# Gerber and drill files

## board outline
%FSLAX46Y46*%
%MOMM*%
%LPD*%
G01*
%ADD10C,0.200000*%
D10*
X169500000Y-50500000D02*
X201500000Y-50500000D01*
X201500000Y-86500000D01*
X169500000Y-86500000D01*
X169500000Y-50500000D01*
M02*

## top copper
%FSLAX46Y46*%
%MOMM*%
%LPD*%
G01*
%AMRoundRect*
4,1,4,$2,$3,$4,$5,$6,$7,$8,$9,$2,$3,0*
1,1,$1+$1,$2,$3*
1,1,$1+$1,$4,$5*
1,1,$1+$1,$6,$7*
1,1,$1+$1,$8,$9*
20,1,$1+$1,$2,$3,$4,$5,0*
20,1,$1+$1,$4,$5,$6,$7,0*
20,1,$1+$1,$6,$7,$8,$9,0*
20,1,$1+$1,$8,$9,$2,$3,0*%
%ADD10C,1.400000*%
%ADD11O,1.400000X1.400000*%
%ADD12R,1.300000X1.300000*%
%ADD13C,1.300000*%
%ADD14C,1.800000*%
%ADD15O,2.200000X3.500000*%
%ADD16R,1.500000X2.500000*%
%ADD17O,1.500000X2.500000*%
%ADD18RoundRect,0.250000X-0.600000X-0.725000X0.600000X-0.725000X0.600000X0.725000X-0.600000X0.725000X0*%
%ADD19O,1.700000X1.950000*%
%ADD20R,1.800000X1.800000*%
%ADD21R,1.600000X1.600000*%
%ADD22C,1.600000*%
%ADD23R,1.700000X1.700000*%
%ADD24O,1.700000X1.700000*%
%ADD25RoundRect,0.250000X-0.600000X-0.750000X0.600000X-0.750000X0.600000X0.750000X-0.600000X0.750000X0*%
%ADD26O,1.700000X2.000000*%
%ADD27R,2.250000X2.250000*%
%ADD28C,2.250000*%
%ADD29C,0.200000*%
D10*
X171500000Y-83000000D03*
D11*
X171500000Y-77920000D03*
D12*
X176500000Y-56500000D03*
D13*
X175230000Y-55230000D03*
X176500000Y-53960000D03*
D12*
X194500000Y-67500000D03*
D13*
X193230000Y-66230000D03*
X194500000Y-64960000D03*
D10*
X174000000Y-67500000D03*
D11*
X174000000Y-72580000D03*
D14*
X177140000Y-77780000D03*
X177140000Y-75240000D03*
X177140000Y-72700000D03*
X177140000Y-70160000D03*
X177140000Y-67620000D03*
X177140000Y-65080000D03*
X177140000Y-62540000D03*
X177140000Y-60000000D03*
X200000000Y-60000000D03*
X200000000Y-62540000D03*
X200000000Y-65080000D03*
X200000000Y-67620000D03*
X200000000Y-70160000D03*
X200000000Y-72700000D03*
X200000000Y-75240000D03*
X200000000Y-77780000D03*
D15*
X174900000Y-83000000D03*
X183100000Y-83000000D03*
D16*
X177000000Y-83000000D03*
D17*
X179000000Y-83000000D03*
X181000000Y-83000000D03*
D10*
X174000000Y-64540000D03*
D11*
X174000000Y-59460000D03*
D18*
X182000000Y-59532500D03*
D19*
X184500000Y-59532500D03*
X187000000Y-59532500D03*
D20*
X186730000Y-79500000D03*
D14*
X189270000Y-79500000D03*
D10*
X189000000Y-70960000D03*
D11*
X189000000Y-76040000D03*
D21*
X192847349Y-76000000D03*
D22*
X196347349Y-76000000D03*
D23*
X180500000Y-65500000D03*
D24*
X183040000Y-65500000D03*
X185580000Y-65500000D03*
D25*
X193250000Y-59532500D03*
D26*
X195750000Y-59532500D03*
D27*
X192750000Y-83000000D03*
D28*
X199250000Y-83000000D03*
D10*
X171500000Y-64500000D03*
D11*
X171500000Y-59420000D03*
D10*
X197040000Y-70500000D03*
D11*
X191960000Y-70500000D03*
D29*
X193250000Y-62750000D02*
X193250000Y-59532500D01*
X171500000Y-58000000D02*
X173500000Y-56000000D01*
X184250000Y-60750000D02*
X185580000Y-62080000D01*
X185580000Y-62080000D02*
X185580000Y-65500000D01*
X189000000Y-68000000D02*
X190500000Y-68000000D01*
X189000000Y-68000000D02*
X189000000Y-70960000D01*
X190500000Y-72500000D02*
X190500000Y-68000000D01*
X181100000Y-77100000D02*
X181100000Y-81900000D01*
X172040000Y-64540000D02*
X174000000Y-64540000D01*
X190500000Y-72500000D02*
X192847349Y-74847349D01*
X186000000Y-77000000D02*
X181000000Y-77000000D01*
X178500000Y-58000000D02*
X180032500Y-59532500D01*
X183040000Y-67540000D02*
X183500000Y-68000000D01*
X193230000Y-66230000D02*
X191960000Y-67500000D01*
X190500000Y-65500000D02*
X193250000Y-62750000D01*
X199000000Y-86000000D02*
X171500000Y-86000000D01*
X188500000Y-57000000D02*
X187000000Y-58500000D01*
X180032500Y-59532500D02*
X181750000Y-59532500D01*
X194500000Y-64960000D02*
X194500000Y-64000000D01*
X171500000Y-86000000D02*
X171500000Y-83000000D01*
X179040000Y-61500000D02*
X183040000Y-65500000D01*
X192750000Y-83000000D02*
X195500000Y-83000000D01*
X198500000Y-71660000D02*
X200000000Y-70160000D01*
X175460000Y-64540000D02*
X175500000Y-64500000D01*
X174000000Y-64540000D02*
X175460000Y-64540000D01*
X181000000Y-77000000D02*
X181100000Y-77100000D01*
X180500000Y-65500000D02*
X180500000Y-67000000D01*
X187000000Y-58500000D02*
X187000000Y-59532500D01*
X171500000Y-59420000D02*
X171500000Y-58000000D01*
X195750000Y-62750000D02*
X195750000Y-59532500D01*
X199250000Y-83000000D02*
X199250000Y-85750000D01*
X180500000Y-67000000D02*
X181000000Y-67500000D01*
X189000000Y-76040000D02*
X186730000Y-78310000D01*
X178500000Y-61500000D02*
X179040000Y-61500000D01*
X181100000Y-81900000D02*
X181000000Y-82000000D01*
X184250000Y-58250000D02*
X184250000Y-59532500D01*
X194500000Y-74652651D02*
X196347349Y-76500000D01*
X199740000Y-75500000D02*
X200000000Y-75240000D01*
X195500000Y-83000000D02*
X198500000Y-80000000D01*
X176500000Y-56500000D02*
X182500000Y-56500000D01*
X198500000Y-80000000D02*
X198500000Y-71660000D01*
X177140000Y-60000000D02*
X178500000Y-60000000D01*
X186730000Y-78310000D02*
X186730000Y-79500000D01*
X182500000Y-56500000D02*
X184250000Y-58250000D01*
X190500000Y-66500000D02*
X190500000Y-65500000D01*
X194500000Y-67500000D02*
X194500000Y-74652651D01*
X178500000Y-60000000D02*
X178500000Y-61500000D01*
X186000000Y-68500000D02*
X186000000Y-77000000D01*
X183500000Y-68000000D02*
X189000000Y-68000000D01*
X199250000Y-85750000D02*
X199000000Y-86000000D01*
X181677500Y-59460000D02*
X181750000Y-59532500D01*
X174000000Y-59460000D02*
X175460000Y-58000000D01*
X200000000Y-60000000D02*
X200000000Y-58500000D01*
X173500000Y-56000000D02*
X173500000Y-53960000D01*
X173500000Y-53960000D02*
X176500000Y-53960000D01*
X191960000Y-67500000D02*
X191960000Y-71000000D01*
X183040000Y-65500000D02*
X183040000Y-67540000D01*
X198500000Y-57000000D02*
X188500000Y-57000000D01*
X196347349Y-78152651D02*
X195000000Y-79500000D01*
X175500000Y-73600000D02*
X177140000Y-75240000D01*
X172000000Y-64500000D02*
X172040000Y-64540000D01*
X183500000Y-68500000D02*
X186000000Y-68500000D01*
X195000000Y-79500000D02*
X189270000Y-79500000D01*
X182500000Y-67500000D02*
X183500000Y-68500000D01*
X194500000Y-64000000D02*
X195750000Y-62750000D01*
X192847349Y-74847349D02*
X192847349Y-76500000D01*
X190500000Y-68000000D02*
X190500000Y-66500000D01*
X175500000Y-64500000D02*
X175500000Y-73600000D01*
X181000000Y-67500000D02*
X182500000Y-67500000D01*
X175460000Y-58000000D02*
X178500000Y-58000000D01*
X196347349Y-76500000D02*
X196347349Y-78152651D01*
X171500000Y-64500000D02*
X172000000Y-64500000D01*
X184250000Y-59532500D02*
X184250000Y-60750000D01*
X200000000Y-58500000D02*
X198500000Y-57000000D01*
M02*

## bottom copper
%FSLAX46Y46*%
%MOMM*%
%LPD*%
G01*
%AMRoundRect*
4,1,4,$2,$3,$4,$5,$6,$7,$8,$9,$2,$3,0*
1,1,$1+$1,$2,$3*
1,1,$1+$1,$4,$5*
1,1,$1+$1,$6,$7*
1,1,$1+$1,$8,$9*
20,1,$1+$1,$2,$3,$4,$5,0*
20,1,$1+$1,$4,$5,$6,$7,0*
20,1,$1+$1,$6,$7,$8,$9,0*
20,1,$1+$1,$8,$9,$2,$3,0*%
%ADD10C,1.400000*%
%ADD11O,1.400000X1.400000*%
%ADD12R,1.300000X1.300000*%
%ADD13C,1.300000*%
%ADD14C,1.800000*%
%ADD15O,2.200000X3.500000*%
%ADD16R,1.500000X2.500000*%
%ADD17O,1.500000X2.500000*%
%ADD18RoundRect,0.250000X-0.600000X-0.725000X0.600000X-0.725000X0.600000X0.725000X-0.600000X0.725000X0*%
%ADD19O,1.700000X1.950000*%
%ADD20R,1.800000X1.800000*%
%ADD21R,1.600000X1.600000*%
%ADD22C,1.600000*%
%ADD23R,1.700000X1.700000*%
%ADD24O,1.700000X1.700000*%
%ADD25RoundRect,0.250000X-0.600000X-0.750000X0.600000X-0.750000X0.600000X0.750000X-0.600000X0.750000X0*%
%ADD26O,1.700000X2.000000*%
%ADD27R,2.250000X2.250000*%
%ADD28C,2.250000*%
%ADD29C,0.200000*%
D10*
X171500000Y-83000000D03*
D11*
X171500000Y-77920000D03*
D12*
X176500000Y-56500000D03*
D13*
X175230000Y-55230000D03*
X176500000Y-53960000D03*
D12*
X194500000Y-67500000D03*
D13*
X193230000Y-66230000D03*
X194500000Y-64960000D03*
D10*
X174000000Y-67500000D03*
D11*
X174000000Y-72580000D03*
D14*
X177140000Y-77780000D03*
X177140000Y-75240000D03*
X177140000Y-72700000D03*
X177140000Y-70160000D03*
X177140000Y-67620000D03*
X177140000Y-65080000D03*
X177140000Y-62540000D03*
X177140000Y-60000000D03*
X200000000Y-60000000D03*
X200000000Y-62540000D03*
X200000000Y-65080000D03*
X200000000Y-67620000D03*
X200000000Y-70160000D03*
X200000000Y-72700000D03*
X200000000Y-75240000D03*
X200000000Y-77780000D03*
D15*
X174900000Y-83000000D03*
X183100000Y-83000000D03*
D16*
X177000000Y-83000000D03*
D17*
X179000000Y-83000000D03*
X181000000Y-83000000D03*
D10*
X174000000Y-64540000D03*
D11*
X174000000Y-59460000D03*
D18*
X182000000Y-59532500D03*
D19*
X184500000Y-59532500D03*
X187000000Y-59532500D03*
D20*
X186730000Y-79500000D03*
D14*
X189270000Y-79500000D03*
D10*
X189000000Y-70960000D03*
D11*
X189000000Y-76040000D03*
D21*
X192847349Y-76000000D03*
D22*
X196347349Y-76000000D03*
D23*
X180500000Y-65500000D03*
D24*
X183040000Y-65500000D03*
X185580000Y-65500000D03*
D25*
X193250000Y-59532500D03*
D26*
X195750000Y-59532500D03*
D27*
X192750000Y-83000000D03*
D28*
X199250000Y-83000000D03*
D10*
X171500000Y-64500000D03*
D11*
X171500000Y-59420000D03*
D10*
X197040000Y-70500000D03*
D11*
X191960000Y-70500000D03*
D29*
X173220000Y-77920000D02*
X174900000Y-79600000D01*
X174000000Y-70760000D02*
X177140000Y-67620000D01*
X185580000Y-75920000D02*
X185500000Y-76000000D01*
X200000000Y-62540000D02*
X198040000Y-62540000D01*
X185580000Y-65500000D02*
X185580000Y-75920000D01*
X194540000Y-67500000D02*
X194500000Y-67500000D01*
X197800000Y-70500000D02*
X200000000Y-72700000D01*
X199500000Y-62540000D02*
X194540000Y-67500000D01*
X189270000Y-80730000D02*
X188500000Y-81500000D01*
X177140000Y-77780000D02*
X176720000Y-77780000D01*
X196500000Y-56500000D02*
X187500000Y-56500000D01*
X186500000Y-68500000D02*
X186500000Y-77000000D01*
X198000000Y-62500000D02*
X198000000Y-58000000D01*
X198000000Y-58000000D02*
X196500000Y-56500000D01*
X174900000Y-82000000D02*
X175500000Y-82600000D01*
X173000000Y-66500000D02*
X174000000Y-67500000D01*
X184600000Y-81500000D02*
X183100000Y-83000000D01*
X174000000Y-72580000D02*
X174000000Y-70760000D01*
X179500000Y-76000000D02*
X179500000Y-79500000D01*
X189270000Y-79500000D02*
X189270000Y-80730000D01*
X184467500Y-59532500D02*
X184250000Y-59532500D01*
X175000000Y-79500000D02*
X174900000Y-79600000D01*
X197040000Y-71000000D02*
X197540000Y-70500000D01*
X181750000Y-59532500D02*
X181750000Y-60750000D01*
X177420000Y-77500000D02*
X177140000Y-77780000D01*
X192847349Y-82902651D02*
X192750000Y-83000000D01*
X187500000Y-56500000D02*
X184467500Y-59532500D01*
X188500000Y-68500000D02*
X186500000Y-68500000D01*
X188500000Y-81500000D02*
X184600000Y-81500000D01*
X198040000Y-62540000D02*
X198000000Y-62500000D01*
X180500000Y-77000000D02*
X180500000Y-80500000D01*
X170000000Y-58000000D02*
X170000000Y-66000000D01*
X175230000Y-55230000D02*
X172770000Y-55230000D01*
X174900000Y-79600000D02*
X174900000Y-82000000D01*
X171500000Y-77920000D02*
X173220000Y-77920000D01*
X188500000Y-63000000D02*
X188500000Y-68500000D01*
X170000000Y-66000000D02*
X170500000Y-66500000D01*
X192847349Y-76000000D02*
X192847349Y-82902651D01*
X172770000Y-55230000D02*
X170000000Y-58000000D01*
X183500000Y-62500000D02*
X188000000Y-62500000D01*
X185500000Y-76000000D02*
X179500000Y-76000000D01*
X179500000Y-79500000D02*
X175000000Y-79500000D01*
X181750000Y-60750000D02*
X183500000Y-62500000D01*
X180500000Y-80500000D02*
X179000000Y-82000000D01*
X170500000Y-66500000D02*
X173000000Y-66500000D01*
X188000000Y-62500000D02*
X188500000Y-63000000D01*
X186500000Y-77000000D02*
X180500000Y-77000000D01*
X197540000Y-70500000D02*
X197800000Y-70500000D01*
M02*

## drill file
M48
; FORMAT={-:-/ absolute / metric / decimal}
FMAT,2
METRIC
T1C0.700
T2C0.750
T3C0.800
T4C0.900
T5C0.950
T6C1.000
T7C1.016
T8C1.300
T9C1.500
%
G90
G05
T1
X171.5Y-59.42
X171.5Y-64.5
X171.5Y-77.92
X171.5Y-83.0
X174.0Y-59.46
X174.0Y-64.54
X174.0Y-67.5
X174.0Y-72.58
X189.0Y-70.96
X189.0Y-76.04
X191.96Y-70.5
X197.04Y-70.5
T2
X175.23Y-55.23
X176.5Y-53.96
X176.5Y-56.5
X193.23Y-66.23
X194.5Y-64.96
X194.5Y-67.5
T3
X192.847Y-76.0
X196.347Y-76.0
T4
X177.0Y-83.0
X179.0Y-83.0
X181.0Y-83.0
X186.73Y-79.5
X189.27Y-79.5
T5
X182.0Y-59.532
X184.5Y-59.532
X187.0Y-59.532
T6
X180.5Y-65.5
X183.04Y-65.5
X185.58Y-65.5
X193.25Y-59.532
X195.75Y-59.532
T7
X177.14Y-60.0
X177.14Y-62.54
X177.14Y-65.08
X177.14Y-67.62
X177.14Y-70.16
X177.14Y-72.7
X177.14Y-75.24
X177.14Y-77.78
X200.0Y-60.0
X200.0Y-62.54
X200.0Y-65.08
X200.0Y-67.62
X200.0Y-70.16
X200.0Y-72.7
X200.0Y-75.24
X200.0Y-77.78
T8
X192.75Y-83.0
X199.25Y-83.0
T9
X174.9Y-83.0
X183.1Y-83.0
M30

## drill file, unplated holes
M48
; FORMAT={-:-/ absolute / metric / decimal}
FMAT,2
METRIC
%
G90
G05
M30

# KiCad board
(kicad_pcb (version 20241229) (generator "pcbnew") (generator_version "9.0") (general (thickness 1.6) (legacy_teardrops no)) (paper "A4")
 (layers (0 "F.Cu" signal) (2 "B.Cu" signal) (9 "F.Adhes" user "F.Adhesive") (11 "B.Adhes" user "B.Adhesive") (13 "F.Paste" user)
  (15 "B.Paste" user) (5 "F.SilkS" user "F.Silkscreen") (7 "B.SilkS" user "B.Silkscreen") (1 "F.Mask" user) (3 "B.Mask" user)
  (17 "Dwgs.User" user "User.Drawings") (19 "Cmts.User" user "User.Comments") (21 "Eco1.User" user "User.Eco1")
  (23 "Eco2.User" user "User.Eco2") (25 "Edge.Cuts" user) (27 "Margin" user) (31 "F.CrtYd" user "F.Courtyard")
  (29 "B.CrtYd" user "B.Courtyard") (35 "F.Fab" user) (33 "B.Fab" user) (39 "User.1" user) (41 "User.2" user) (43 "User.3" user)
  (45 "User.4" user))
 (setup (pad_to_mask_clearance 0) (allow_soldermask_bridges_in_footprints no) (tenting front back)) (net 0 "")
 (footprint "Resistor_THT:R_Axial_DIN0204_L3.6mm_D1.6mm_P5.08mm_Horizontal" (layer "F.Cu") (at 171.5 83 90)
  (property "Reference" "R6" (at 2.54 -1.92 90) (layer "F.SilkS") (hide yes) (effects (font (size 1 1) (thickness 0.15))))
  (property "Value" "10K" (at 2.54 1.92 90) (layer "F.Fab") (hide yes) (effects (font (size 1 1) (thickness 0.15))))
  (pad "1" thru_hole circle (at 0 0 90) (size 1.4 1.4) (drill 0.7) (layers "*.Cu" "*.Mask") (remove_unused_layers no))
  (pad "2" thru_hole oval (at 5.08 0 90) (size 1.4 1.4) (drill 0.7) (layers "*.Cu" "*.Mask") (remove_unused_layers no)))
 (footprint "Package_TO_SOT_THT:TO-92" (layer "F.Cu") (at 176.5 56.5 90)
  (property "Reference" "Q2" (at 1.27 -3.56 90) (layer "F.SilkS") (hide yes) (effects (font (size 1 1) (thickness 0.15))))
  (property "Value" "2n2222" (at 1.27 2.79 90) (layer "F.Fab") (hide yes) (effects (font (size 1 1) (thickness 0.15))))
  (pad "1" thru_hole rect (at 0 0 90) (size 1.3 1.3) (drill 0.75) (layers "*.Cu" "*.Mask") (remove_unused_layers no))
  (pad "2" thru_hole circle (at 1.27 -1.27 90) (size 1.3 1.3) (drill 0.75) (layers "*.Cu" "*.Mask") (remove_unused_layers no))
  (pad "3" thru_hole circle (at 2.54 0 90) (size 1.3 1.3) (drill 0.75) (layers "*.Cu" "*.Mask") (remove_unused_layers no)))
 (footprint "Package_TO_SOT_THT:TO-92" (layer "F.Cu") (at 194.5 67.5 90)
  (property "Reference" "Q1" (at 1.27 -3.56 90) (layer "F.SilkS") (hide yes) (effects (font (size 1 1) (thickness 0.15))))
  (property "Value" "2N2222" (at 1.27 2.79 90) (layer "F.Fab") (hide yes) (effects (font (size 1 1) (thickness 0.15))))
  (pad "1" thru_hole rect (at 0 0 90) (size 1.3 1.3) (drill 0.75) (layers "*.Cu" "*.Mask") (remove_unused_layers no))
  (pad "2" thru_hole circle (at 1.27 -1.27 90) (size 1.3 1.3) (drill 0.75) (layers "*.Cu" "*.Mask") (remove_unused_layers no))
  (pad "3" thru_hole circle (at 2.54 0 90) (size 1.3 1.3) (drill 0.75) (layers "*.Cu" "*.Mask") (remove_unused_layers no)))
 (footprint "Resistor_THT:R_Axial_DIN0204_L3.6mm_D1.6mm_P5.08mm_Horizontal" (layer "F.Cu") (at 174 67.5 -90)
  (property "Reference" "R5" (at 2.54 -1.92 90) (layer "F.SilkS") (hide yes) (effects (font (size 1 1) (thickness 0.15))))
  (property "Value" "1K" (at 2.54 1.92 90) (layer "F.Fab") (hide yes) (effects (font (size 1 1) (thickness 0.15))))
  (pad "1" thru_hole circle (at 0 0 270) (size 1.4 1.4) (drill 0.7) (layers "*.Cu" "*.Mask") (remove_unused_layers no))
  (pad "2" thru_hole oval (at 5.08 0 270) (size 1.4 1.4) (drill 0.7) (layers "*.Cu" "*.Mask") (remove_unused_layers no)))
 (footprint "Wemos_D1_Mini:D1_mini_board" (layer "F.Cu") (at 188.57 70.16)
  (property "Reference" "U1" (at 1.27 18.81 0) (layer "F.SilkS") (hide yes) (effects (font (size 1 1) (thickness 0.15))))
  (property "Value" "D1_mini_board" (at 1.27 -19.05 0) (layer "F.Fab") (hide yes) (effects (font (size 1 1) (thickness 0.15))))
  (pad "1" thru_hole circle (at -11.43 7.62) (size 1.8 1.8) (drill 1.016) (layers "*.Cu" "*.Mask" "F.SilkS") (remove_unused_layers no))
  (pad "2" thru_hole circle (at -11.43 5.08) (size 1.8 1.8) (drill 1.016) (layers "*.Cu" "*.Mask" "F.SilkS") (remove_unused_layers no))
  (pad "3" thru_hole circle (at -11.43 2.54) (size 1.8 1.8) (drill 1.016) (layers "*.Cu" "*.Mask" "F.SilkS") (remove_unused_layers no))
  (pad "4" thru_hole circle (at -11.43 0) (size 1.8 1.8) (drill 1.016) (layers "*.Cu" "*.Mask" "F.SilkS") (remove_unused_layers no))
  (pad "5" thru_hole circle (at -11.43 -2.54) (size 1.8 1.8) (drill 1.016) (layers "*.Cu" "*.Mask" "F.SilkS") (remove_unused_layers no))
  (pad "6" thru_hole circle (at -11.43 -5.08) (size 1.8 1.8) (drill 1.016) (layers "*.Cu" "*.Mask" "F.SilkS") (remove_unused_layers no))
  (pad "7" thru_hole circle (at -11.43 -7.62) (size 1.8 1.8) (drill 1.016) (layers "*.Cu" "*.Mask" "F.SilkS") (remove_unused_layers no))
  (pad "8" thru_hole circle (at -11.43 -10.16) (size 1.8 1.8) (drill 1.016) (layers "*.Cu" "*.Mask" "F.SilkS") (remove_unused_layers no))
  (pad "9" thru_hole circle (at 11.43 -10.16) (size 1.8 1.8) (drill 1.016) (layers "*.Cu" "*.Mask" "F.SilkS") (remove_unused_layers no))
  (pad "10" thru_hole circle (at 11.43 -7.62) (size 1.8 1.8) (drill 1.016) (layers "*.Cu" "*.Mask" "F.SilkS") (remove_unused_layers no))
  (pad "11" thru_hole circle (at 11.43 -5.08) (size 1.8 1.8) (drill 1.016) (layers "*.Cu" "*.Mask" "F.SilkS") (remove_unused_layers no))
  (pad "12" thru_hole circle (at 11.43 -2.54) (size 1.8 1.8) (drill 1.016) (layers "*.Cu" "*.Mask" "F.SilkS") (remove_unused_layers no))
  (pad "13" thru_hole circle (at 11.43 0) (size 1.8 1.8) (drill 1.016) (layers "*.Cu" "*.Mask" "F.SilkS") (remove_unused_layers no))
  (pad "14" thru_hole circle (at 11.43 2.54) (size 1.8 1.8) (drill 1.016) (layers "*.Cu" "*.Mask" "F.SilkS") (remove_unused_layers no))
  (pad "15" thru_hole circle (at 11.43 5.08) (size 1.8 1.8) (drill 1.016) (layers "*.Cu" "*.Mask" "F.SilkS") (remove_unused_layers no))
  (pad "16" thru_hole circle (at 11.43 7.62) (size 1.8 1.8) (drill 1.016) (layers "*.Cu" "*.Mask" "F.SilkS") (remove_unused_layers no)))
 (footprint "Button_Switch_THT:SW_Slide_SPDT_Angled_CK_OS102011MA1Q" (layer "F.Cu") (at 177 83)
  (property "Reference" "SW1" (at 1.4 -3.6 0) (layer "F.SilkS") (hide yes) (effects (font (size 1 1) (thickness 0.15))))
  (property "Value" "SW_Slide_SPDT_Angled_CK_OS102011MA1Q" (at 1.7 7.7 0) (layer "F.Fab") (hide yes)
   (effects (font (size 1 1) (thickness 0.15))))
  (pad "" thru_hole oval (at -2.1 0) (size 2.2 3.5) (drill 1.5) (layers "*.Cu" "*.Mask") (remove_unused_layers no))
  (pad "" thru_hole oval (at 6.1 0) (size 2.2 3.5) (drill 1.5) (layers "*.Cu" "*.Mask") (remove_unused_layers no))
  (pad "1" thru_hole rect (at 0 0) (size 1.5 2.5) (drill 0.9) (layers "*.Cu" "*.Mask") (remove_unused_layers no))
  (pad "2" thru_hole oval (at 2 0) (size 1.5 2.5) (drill 0.9) (layers "*.Cu" "*.Mask") (remove_unused_layers no))
  (pad "3" thru_hole oval (at 4 0) (size 1.5 2.5) (drill 0.9) (layers "*.Cu" "*.Mask") (remove_unused_layers no)))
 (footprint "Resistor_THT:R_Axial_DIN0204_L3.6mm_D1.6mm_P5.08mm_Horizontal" (layer "F.Cu") (at 174 64.54 90)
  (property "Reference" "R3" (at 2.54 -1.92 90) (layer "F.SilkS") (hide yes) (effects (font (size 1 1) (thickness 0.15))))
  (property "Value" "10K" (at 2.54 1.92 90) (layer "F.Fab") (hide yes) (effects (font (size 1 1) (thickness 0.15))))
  (pad "1" thru_hole circle (at 0 0 90) (size 1.4 1.4) (drill 0.7) (layers "*.Cu" "*.Mask") (remove_unused_layers no))
  (pad "2" thru_hole oval (at 5.08 0 90) (size 1.4 1.4) (drill 0.7) (layers "*.Cu" "*.Mask") (remove_unused_layers no)))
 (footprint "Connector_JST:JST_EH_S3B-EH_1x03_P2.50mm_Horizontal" (layer "F.Cu") (at 182 59.5325)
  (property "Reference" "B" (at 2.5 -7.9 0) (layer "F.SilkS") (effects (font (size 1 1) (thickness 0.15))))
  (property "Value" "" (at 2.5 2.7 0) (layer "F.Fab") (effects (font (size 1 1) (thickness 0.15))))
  (pad "1" thru_hole roundrect (at 0 0) (size 1.7 1.95) (drill 0.95) (layers "*.Cu" "*.Mask") (remove_unused_layers no)
   (roundrect_rratio 0.147059))
  (pad "2" thru_hole oval (at 2.5 0) (size 1.7 1.95) (drill 0.95) (layers "*.Cu" "*.Mask") (remove_unused_layers no))
  (pad "3" thru_hole oval (at 5 0) (size 1.7 1.95) (drill 0.95) (layers "*.Cu" "*.Mask") (remove_unused_layers no)))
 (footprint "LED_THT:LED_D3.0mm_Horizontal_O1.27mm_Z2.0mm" (layer "F.Cu") (at 186.73 79.5)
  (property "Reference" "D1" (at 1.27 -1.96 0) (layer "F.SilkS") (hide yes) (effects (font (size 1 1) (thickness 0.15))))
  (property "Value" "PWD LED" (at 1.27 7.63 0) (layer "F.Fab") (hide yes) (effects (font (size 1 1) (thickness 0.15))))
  (pad "1" thru_hole rect (at 0 0) (size 1.8 1.8) (drill 0.9) (layers "*.Cu" "*.Mask") (remove_unused_layers no))
  (pad "2" thru_hole circle (at 2.54 0) (size 1.8 1.8) (drill 0.9) (layers "*.Cu" "*.Mask") (remove_unused_layers no)))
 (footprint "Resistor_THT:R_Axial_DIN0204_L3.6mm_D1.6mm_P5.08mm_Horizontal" (layer "F.Cu") (at 189 70.96 -90)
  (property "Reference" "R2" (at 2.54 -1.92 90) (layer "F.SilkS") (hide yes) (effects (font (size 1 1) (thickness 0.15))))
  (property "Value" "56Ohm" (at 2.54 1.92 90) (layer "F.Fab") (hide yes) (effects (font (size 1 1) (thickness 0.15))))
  (pad "1" thru_hole circle (at 0 0 270) (size 1.4 1.4) (drill 0.7) (layers "*.Cu" "*.Mask") (remove_unused_layers no))
  (pad "2" thru_hole oval (at 5.08 0 270) (size 1.4 1.4) (drill 0.7) (layers "*.Cu" "*.Mask") (remove_unused_layers no)))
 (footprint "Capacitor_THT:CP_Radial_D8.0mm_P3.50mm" (layer "F.Cu") (at 192.847349 76)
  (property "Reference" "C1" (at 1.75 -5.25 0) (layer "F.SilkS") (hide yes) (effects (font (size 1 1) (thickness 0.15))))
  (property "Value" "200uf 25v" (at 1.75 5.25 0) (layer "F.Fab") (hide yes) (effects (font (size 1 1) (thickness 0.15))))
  (pad "1" thru_hole rect (at 0 0) (size 1.6 1.6) (drill 0.8) (layers "*.Cu" "*.Mask") (remove_unused_layers no))
  (pad "2" thru_hole circle (at 3.5 0) (size 1.6 1.6) (drill 0.8) (layers "*.Cu" "*.Mask") (remove_unused_layers no)))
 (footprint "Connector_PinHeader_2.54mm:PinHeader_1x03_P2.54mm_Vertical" (layer "F.Cu") (at 180.5 65.5 90)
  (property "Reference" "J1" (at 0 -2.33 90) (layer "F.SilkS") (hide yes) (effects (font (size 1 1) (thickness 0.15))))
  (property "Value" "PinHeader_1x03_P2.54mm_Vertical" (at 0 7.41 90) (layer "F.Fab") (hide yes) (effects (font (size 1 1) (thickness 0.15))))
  (pad "1" thru_hole rect (at 0 0 90) (size 1.7 1.7) (drill 1) (layers "*.Cu" "*.Mask") (remove_unused_layers no))
  (pad "2" thru_hole oval (at 0 2.54 90) (size 1.7 1.7) (drill 1) (layers "*.Cu" "*.Mask") (remove_unused_layers no))
  (pad "3" thru_hole oval (at 0 5.08 90) (size 1.7 1.7) (drill 1) (layers "*.Cu" "*.Mask") (remove_unused_layers no)))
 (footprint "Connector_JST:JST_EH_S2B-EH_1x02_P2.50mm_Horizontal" (layer "F.Cu") (at 193.25 59.5325)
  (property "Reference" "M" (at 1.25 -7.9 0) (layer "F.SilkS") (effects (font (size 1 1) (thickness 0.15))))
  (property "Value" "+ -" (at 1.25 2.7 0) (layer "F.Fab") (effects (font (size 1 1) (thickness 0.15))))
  (pad "1" thru_hole roundrect (at 0 0) (size 1.7 2) (drill 1) (layers "*.Cu" "*.Mask") (remove_unused_layers no)
   (roundrect_rratio 0.147059))
  (pad "2" thru_hole oval (at 2.5 0) (size 1.7 2) (drill 1) (layers "*.Cu" "*.Mask") (remove_unused_layers no)))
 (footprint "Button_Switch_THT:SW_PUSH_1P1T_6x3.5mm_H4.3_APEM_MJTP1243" (layer "F.Cu") (at 192.75 83)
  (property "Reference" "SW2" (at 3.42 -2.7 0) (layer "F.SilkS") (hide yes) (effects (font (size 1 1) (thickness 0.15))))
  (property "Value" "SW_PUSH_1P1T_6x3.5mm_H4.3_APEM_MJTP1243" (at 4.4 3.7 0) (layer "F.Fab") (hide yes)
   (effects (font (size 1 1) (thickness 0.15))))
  (pad "1" thru_hole rect (at 0 0 90) (size 2.25 2.25) (drill 1.3) (layers "*.Cu" "*.Mask") (remove_unused_layers no))
  (pad "2" thru_hole circle (at 6.5 0 90) (size 2.25 2.25) (drill 1.3) (layers "*.Cu" "*.Mask") (remove_unused_layers no)))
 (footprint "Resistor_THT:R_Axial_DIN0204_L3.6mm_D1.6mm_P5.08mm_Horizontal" (layer "F.Cu") (at 171.5 64.5 90)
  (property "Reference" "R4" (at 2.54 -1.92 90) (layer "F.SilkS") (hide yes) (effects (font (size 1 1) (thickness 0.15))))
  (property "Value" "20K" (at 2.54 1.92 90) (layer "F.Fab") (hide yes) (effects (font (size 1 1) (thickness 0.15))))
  (pad "1" thru_hole circle (at 0 0 90) (size 1.4 1.4) (drill 0.7) (layers "*.Cu" "*.Mask") (remove_unused_layers no))
  (pad "2" thru_hole oval (at 5.08 0 90) (size 1.4 1.4) (drill 0.7) (layers "*.Cu" "*.Mask") (remove_unused_layers no)))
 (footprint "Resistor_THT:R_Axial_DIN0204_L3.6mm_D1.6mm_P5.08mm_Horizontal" (layer "F.Cu") (at 197.04 70.5 180)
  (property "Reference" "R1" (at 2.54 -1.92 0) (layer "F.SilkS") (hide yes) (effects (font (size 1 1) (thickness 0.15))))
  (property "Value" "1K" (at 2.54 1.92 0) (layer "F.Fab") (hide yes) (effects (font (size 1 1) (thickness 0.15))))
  (pad "1" thru_hole circle (at 0 0 180) (size 1.4 1.4) (drill 0.7) (layers "*.Cu" "*.Mask") (remove_unused_layers no))
  (pad "2" thru_hole oval (at 5.08 0 180) (size 1.4 1.4) (drill 0.7) (layers "*.Cu" "*.Mask") (remove_unused_layers no)))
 (gr_rect (start 169.5 50.5) (end 201.5 86.5) (stroke (width 0.2) (type solid)) (fill no) (layer "Edge.Cuts"))
 (segment (start 193.25 62.75) (end 193.25 59.5325) (width 0.2) (layer "F.Cu") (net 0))
 (segment (start 171.5 58) (end 173.5 56) (width 0.2) (layer "F.Cu") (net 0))
 (segment (start 184.25 60.75) (end 185.58 62.08) (width 0.2) (layer "F.Cu") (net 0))
 (segment (start 185.58 62.08) (end 185.58 65.5) (width 0.2) (layer "F.Cu") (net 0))
 (segment (start 189 68) (end 190.5 68) (width 0.2) (layer "F.Cu") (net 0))
 (segment (start 189 68) (end 189 70.96) (width 0.2) (layer "F.Cu") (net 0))
 (segment (start 190.5 72.5) (end 190.5 68) (width 0.2) (layer "F.Cu") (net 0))
 (segment (start 181.1 77.1) (end 181.1 81.9) (width 0.2) (layer "F.Cu") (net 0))
 (segment (start 172.04 64.54) (end 174 64.54) (width 0.2) (layer "F.Cu") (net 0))
 (segment (start 190.5 72.5) (end 192.847349 74.847349) (width 0.2) (layer "F.Cu") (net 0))
 (segment (start 186 77) (end 181 77) (width 0.2) (layer "F.Cu") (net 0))
 (segment (start 178.5 58) (end 180.0325 59.5325) (width 0.2) (layer "F.Cu") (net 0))
 (segment (start 183.04 67.54) (end 183.5 68) (width 0.2) (layer "F.Cu") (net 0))
 (segment (start 193.23 66.23) (end 191.96 67.5) (width 0.2) (layer "F.Cu") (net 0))
 (segment (start 190.5 65.5) (end 193.25 62.75) (width 0.2) (layer "F.Cu") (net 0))
 (segment (start 199 86) (end 171.5 86) (width 0.2) (layer "F.Cu") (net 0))
 (segment (start 188.5 57) (end 187 58.5) (width 0.2) (layer "F.Cu") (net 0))
 (segment (start 180.0325 59.5325) (end 181.75 59.5325) (width 0.2) (layer "F.Cu") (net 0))
 (segment (start 194.5 64.96) (end 194.5 64) (width 0.2) (layer "F.Cu") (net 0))
 (segment (start 171.5 86) (end 171.5 83) (width 0.2) (layer "F.Cu") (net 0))
 (segment (start 179.04 61.5) (end 183.04 65.5) (width 0.2) (layer "F.Cu") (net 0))
 (segment (start 192.75 83) (end 195.5 83) (width 0.2) (layer "F.Cu") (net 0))
 (segment (start 198.5 71.66) (end 200 70.16) (width 0.2) (layer "F.Cu") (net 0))
 (segment (start 175.46 64.54) (end 175.5 64.5) (width 0.2) (layer "F.Cu") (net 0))
 (segment (start 174 64.54) (end 175.46 64.54) (width 0.2) (layer "F.Cu") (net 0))
 (segment (start 181 77) (end 181.1 77.1) (width 0.2) (layer "F.Cu") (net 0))
 (segment (start 180.5 65.5) (end 180.5 67) (width 0.2) (layer "F.Cu") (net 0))
 (segment (start 187 58.5) (end 187 59.5325) (width 0.2) (layer "F.Cu") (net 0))
 (segment (start 171.5 59.42) (end 171.5 58) (width 0.2) (layer "F.Cu") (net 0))
 (segment (start 195.75 62.75) (end 195.75 59.5325) (width 0.2) (layer "F.Cu") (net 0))
 (segment (start 199.25 83) (end 199.25 85.75) (width 0.2) (layer "F.Cu") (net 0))
 (segment (start 180.5 67) (end 181 67.5) (width 0.2) (layer "F.Cu") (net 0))
 (segment (start 189 76.04) (end 186.73 78.31) (width 0.2) (layer "F.Cu") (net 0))
 (segment (start 178.5 61.5) (end 179.04 61.5) (width 0.2) (layer "F.Cu") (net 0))
 (segment (start 181.1 81.9) (end 181 82) (width 0.2) (layer "F.Cu") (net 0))
 (segment (start 184.25 58.25) (end 184.25 59.5325) (width 0.2) (layer "F.Cu") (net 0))
 (segment (start 194.5 74.652651) (end 196.347349 76.5) (width 0.2) (layer "F.Cu") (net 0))
 (segment (start 199.74 75.5) (end 200 75.24) (width 0.2) (layer "F.Cu") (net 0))
 (segment (start 195.5 83) (end 198.5 80) (width 0.2) (layer "F.Cu") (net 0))
 (segment (start 176.5 56.5) (end 182.5 56.5) (width 0.2) (layer "F.Cu") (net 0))
 (segment (start 198.5 80) (end 198.5 71.66) (width 0.2) (layer "F.Cu") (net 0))
 (segment (start 177.14 60) (end 178.5 60) (width 0.2) (layer "F.Cu") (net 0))
 (segment (start 186.73 78.31) (end 186.73 79.5) (width 0.2) (layer "F.Cu") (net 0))
 (segment (start 182.5 56.5) (end 184.25 58.25) (width 0.2) (layer "F.Cu") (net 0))
 (segment (start 190.5 66.5) (end 190.5 65.5) (width 0.2) (layer "F.Cu") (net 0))
 (segment (start 194.5 67.5) (end 194.5 74.652651) (width 0.2) (layer "F.Cu") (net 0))
 (segment (start 178.5 60) (end 178.5 61.5) (width 0.2) (layer "F.Cu") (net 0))
 (segment (start 186 68.5) (end 186 77) (width 0.2) (layer "F.Cu") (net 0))
 (segment (start 183.5 68) (end 189 68) (width 0.2) (layer "F.Cu") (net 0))
 (segment (start 199.25 85.75) (end 199 86) (width 0.2) (layer "F.Cu") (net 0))
 (segment (start 181.6775 59.46) (end 181.75 59.5325) (width 0.2) (layer "F.Cu") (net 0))
 (segment (start 174 59.46) (end 175.46 58) (width 0.2) (layer "F.Cu") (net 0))
 (segment (start 200 60) (end 200 58.5) (width 0.2) (layer "F.Cu") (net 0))
 (segment (start 173.5 56) (end 173.5 53.96) (width 0.2) (layer "F.Cu") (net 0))
 (segment (start 173.5 53.96) (end 176.5 53.96) (width 0.2) (layer "F.Cu") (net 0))
 (segment (start 191.96 67.5) (end 191.96 71) (width 0.2) (layer "F.Cu") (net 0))
 (segment (start 183.04 65.5) (end 183.04 67.54) (width 0.2) (layer "F.Cu") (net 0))
 (segment (start 198.5 57) (end 188.5 57) (width 0.2) (layer "F.Cu") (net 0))
 (segment (start 196.347349 78.152651) (end 195 79.5) (width 0.2) (layer "F.Cu") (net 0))
 (segment (start 175.5 73.6) (end 177.14 75.24) (width 0.2) (layer "F.Cu") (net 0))
 (segment (start 172 64.5) (end 172.04 64.54) (width 0.2) (layer "F.Cu") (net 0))
 (segment (start 183.5 68.5) (end 186 68.5) (width 0.2) (layer "F.Cu") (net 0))
 (segment (start 195 79.5) (end 189.27 79.5) (width 0.2) (layer "F.Cu") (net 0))
 (segment (start 182.5 67.5) (end 183.5 68.5) (width 0.2) (layer "F.Cu") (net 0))
 (segment (start 194.5 64) (end 195.75 62.75) (width 0.2) (layer "F.Cu") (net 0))
 (segment (start 192.847349 74.847349) (end 192.847349 76.5) (width 0.2) (layer "F.Cu") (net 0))
 (segment (start 190.5 68) (end 190.5 66.5) (width 0.2) (layer "F.Cu") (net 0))
 (segment (start 175.5 64.5) (end 175.5 73.6) (width 0.2) (layer "F.Cu") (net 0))
 (segment (start 181 67.5) (end 182.5 67.5) (width 0.2) (layer "F.Cu") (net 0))
 (segment (start 175.46 58) (end 178.5 58) (width 0.2) (layer "F.Cu") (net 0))
 (segment (start 196.347349 76.5) (end 196.347349 78.152651) (width 0.2) (layer "F.Cu") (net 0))
 (segment (start 171.5 64.5) (end 172 64.5) (width 0.2) (layer "F.Cu") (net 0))
 (segment (start 184.25 59.5325) (end 184.25 60.75) (width 0.2) (layer "F.Cu") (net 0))
 (segment (start 200 58.5) (end 198.5 57) (width 0.2) (layer "F.Cu") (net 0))
 (segment (start 173.22 77.92) (end 174.9 79.6) (width 0.2) (layer "B.Cu") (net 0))
 (segment (start 174 70.76) (end 177.14 67.62) (width 0.2) (layer "B.Cu") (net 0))
 (segment (start 185.58 75.92) (end 185.5 76) (width 0.2) (layer "B.Cu") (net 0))
 (segment (start 200 62.54) (end 198.04 62.54) (width 0.2) (layer "B.Cu") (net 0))
 (segment (start 185.58 65.5) (end 185.58 75.92) (width 0.2) (layer "B.Cu") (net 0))
 (segment (start 194.54 67.5) (end 194.5 67.5) (width 0.2) (layer "B.Cu") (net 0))
 (segment (start 197.8 70.5) (end 200 72.7) (width 0.2) (layer "B.Cu") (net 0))
 (segment (start 199.5 62.54) (end 194.54 67.5) (width 0.2) (layer "B.Cu") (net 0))
 (segment (start 189.27 80.73) (end 188.5 81.5) (width 0.2) (layer "B.Cu") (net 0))
 (segment (start 177.14 77.78) (end 176.72 77.78) (width 0.2) (layer "B.Cu") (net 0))
 (segment (start 196.5 56.5) (end 187.5 56.5) (width 0.2) (layer "B.Cu") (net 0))
 (segment (start 186.5 68.5) (end 186.5 77) (width 0.2) (layer "B.Cu") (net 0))
 (segment (start 198 62.5) (end 198 58) (width 0.2) (layer "B.Cu") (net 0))
 (segment (start 198 58) (end 196.5 56.5) (width 0.2) (layer "B.Cu") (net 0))
 (segment (start 174.9 82) (end 175.5 82.6) (width 0.2) (layer "B.Cu") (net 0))
 (segment (start 173 66.5) (end 174 67.5) (width 0.2) (layer "B.Cu") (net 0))
 (segment (start 184.6 81.5) (end 183.1 83) (width 0.2) (layer "B.Cu") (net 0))
 (segment (start 174 72.58) (end 174 70.76) (width 0.2) (layer "B.Cu") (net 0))
 (segment (start 179.5 76) (end 179.5 79.5) (width 0.2) (layer "B.Cu") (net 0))
 (segment (start 189.27 79.5) (end 189.27 80.73) (width 0.2) (layer "B.Cu") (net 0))
 (segment (start 184.4675 59.5325) (end 184.25 59.5325) (width 0.2) (layer "B.Cu") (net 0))
 (segment (start 175 79.5) (end 174.9 79.6) (width 0.2) (layer "B.Cu") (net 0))
 (segment (start 197.04 71) (end 197.54 70.5) (width 0.2) (layer "B.Cu") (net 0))
 (segment (start 181.75 59.5325) (end 181.75 60.75) (width 0.2) (layer "B.Cu") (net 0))
 (segment (start 177.42 77.5) (end 177.14 77.78) (width 0.2) (layer "B.Cu") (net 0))
 (segment (start 192.847349 82.902651) (end 192.75 83) (width 0.2) (layer "B.Cu") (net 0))
 (segment (start 187.5 56.5) (end 184.4675 59.5325) (width 0.2) (layer "B.Cu") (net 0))
 (segment (start 188.5 68.5) (end 186.5 68.5) (width 0.2) (layer "B.Cu") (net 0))
 (segment (start 188.5 81.5) (end 184.6 81.5) (width 0.2) (layer "B.Cu") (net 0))
 (segment (start 198.04 62.54) (end 198 62.5) (width 0.2) (layer "B.Cu") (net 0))
 (segment (start 180.5 77) (end 180.5 80.5) (width 0.2) (layer "B.Cu") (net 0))
 (segment (start 170 58) (end 170 66) (width 0.2) (layer "B.Cu") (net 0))
 (segment (start 175.23 55.23) (end 172.77 55.23) (width 0.2) (layer "B.Cu") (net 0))
 (segment (start 174.9 79.6) (end 174.9 82) (width 0.2) (layer "B.Cu") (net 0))
 (segment (start 171.5 77.92) (end 173.22 77.92) (width 0.2) (layer "B.Cu") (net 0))
 (segment (start 188.5 63) (end 188.5 68.5) (width 0.2) (layer "B.Cu") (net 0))
 (segment (start 170 66) (end 170.5 66.5) (width 0.2) (layer "B.Cu") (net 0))
 (segment (start 192.847349 76) (end 192.847349 82.902651) (width 0.2) (layer "B.Cu") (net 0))
 (segment (start 172.77 55.23) (end 170 58) (width 0.2) (layer "B.Cu") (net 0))
 (segment (start 183.5 62.5) (end 188 62.5) (width 0.2) (layer "B.Cu") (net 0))
 (segment (start 185.5 76) (end 179.5 76) (width 0.2) (layer "B.Cu") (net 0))
 (segment (start 179.5 79.5) (end 175 79.5) (width 0.2) (layer "B.Cu") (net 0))
 (segment (start 181.75 60.75) (end 183.5 62.5) (width 0.2) (layer "B.Cu") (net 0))
 (segment (start 180.5 80.5) (end 179 82) (width 0.2) (layer "B.Cu") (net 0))
 (segment (start 170.5 66.5) (end 173 66.5) (width 0.2) (layer "B.Cu") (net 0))
 (segment (start 188 62.5) (end 188.5 63) (width 0.2) (layer "B.Cu") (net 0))
 (segment (start 186.5 77) (end 180.5 77) (width 0.2) (layer "B.Cu") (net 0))
 (segment (start 197.54 70.5) (end 197.8 70.5) (width 0.2) (layer "B.Cu") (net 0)))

